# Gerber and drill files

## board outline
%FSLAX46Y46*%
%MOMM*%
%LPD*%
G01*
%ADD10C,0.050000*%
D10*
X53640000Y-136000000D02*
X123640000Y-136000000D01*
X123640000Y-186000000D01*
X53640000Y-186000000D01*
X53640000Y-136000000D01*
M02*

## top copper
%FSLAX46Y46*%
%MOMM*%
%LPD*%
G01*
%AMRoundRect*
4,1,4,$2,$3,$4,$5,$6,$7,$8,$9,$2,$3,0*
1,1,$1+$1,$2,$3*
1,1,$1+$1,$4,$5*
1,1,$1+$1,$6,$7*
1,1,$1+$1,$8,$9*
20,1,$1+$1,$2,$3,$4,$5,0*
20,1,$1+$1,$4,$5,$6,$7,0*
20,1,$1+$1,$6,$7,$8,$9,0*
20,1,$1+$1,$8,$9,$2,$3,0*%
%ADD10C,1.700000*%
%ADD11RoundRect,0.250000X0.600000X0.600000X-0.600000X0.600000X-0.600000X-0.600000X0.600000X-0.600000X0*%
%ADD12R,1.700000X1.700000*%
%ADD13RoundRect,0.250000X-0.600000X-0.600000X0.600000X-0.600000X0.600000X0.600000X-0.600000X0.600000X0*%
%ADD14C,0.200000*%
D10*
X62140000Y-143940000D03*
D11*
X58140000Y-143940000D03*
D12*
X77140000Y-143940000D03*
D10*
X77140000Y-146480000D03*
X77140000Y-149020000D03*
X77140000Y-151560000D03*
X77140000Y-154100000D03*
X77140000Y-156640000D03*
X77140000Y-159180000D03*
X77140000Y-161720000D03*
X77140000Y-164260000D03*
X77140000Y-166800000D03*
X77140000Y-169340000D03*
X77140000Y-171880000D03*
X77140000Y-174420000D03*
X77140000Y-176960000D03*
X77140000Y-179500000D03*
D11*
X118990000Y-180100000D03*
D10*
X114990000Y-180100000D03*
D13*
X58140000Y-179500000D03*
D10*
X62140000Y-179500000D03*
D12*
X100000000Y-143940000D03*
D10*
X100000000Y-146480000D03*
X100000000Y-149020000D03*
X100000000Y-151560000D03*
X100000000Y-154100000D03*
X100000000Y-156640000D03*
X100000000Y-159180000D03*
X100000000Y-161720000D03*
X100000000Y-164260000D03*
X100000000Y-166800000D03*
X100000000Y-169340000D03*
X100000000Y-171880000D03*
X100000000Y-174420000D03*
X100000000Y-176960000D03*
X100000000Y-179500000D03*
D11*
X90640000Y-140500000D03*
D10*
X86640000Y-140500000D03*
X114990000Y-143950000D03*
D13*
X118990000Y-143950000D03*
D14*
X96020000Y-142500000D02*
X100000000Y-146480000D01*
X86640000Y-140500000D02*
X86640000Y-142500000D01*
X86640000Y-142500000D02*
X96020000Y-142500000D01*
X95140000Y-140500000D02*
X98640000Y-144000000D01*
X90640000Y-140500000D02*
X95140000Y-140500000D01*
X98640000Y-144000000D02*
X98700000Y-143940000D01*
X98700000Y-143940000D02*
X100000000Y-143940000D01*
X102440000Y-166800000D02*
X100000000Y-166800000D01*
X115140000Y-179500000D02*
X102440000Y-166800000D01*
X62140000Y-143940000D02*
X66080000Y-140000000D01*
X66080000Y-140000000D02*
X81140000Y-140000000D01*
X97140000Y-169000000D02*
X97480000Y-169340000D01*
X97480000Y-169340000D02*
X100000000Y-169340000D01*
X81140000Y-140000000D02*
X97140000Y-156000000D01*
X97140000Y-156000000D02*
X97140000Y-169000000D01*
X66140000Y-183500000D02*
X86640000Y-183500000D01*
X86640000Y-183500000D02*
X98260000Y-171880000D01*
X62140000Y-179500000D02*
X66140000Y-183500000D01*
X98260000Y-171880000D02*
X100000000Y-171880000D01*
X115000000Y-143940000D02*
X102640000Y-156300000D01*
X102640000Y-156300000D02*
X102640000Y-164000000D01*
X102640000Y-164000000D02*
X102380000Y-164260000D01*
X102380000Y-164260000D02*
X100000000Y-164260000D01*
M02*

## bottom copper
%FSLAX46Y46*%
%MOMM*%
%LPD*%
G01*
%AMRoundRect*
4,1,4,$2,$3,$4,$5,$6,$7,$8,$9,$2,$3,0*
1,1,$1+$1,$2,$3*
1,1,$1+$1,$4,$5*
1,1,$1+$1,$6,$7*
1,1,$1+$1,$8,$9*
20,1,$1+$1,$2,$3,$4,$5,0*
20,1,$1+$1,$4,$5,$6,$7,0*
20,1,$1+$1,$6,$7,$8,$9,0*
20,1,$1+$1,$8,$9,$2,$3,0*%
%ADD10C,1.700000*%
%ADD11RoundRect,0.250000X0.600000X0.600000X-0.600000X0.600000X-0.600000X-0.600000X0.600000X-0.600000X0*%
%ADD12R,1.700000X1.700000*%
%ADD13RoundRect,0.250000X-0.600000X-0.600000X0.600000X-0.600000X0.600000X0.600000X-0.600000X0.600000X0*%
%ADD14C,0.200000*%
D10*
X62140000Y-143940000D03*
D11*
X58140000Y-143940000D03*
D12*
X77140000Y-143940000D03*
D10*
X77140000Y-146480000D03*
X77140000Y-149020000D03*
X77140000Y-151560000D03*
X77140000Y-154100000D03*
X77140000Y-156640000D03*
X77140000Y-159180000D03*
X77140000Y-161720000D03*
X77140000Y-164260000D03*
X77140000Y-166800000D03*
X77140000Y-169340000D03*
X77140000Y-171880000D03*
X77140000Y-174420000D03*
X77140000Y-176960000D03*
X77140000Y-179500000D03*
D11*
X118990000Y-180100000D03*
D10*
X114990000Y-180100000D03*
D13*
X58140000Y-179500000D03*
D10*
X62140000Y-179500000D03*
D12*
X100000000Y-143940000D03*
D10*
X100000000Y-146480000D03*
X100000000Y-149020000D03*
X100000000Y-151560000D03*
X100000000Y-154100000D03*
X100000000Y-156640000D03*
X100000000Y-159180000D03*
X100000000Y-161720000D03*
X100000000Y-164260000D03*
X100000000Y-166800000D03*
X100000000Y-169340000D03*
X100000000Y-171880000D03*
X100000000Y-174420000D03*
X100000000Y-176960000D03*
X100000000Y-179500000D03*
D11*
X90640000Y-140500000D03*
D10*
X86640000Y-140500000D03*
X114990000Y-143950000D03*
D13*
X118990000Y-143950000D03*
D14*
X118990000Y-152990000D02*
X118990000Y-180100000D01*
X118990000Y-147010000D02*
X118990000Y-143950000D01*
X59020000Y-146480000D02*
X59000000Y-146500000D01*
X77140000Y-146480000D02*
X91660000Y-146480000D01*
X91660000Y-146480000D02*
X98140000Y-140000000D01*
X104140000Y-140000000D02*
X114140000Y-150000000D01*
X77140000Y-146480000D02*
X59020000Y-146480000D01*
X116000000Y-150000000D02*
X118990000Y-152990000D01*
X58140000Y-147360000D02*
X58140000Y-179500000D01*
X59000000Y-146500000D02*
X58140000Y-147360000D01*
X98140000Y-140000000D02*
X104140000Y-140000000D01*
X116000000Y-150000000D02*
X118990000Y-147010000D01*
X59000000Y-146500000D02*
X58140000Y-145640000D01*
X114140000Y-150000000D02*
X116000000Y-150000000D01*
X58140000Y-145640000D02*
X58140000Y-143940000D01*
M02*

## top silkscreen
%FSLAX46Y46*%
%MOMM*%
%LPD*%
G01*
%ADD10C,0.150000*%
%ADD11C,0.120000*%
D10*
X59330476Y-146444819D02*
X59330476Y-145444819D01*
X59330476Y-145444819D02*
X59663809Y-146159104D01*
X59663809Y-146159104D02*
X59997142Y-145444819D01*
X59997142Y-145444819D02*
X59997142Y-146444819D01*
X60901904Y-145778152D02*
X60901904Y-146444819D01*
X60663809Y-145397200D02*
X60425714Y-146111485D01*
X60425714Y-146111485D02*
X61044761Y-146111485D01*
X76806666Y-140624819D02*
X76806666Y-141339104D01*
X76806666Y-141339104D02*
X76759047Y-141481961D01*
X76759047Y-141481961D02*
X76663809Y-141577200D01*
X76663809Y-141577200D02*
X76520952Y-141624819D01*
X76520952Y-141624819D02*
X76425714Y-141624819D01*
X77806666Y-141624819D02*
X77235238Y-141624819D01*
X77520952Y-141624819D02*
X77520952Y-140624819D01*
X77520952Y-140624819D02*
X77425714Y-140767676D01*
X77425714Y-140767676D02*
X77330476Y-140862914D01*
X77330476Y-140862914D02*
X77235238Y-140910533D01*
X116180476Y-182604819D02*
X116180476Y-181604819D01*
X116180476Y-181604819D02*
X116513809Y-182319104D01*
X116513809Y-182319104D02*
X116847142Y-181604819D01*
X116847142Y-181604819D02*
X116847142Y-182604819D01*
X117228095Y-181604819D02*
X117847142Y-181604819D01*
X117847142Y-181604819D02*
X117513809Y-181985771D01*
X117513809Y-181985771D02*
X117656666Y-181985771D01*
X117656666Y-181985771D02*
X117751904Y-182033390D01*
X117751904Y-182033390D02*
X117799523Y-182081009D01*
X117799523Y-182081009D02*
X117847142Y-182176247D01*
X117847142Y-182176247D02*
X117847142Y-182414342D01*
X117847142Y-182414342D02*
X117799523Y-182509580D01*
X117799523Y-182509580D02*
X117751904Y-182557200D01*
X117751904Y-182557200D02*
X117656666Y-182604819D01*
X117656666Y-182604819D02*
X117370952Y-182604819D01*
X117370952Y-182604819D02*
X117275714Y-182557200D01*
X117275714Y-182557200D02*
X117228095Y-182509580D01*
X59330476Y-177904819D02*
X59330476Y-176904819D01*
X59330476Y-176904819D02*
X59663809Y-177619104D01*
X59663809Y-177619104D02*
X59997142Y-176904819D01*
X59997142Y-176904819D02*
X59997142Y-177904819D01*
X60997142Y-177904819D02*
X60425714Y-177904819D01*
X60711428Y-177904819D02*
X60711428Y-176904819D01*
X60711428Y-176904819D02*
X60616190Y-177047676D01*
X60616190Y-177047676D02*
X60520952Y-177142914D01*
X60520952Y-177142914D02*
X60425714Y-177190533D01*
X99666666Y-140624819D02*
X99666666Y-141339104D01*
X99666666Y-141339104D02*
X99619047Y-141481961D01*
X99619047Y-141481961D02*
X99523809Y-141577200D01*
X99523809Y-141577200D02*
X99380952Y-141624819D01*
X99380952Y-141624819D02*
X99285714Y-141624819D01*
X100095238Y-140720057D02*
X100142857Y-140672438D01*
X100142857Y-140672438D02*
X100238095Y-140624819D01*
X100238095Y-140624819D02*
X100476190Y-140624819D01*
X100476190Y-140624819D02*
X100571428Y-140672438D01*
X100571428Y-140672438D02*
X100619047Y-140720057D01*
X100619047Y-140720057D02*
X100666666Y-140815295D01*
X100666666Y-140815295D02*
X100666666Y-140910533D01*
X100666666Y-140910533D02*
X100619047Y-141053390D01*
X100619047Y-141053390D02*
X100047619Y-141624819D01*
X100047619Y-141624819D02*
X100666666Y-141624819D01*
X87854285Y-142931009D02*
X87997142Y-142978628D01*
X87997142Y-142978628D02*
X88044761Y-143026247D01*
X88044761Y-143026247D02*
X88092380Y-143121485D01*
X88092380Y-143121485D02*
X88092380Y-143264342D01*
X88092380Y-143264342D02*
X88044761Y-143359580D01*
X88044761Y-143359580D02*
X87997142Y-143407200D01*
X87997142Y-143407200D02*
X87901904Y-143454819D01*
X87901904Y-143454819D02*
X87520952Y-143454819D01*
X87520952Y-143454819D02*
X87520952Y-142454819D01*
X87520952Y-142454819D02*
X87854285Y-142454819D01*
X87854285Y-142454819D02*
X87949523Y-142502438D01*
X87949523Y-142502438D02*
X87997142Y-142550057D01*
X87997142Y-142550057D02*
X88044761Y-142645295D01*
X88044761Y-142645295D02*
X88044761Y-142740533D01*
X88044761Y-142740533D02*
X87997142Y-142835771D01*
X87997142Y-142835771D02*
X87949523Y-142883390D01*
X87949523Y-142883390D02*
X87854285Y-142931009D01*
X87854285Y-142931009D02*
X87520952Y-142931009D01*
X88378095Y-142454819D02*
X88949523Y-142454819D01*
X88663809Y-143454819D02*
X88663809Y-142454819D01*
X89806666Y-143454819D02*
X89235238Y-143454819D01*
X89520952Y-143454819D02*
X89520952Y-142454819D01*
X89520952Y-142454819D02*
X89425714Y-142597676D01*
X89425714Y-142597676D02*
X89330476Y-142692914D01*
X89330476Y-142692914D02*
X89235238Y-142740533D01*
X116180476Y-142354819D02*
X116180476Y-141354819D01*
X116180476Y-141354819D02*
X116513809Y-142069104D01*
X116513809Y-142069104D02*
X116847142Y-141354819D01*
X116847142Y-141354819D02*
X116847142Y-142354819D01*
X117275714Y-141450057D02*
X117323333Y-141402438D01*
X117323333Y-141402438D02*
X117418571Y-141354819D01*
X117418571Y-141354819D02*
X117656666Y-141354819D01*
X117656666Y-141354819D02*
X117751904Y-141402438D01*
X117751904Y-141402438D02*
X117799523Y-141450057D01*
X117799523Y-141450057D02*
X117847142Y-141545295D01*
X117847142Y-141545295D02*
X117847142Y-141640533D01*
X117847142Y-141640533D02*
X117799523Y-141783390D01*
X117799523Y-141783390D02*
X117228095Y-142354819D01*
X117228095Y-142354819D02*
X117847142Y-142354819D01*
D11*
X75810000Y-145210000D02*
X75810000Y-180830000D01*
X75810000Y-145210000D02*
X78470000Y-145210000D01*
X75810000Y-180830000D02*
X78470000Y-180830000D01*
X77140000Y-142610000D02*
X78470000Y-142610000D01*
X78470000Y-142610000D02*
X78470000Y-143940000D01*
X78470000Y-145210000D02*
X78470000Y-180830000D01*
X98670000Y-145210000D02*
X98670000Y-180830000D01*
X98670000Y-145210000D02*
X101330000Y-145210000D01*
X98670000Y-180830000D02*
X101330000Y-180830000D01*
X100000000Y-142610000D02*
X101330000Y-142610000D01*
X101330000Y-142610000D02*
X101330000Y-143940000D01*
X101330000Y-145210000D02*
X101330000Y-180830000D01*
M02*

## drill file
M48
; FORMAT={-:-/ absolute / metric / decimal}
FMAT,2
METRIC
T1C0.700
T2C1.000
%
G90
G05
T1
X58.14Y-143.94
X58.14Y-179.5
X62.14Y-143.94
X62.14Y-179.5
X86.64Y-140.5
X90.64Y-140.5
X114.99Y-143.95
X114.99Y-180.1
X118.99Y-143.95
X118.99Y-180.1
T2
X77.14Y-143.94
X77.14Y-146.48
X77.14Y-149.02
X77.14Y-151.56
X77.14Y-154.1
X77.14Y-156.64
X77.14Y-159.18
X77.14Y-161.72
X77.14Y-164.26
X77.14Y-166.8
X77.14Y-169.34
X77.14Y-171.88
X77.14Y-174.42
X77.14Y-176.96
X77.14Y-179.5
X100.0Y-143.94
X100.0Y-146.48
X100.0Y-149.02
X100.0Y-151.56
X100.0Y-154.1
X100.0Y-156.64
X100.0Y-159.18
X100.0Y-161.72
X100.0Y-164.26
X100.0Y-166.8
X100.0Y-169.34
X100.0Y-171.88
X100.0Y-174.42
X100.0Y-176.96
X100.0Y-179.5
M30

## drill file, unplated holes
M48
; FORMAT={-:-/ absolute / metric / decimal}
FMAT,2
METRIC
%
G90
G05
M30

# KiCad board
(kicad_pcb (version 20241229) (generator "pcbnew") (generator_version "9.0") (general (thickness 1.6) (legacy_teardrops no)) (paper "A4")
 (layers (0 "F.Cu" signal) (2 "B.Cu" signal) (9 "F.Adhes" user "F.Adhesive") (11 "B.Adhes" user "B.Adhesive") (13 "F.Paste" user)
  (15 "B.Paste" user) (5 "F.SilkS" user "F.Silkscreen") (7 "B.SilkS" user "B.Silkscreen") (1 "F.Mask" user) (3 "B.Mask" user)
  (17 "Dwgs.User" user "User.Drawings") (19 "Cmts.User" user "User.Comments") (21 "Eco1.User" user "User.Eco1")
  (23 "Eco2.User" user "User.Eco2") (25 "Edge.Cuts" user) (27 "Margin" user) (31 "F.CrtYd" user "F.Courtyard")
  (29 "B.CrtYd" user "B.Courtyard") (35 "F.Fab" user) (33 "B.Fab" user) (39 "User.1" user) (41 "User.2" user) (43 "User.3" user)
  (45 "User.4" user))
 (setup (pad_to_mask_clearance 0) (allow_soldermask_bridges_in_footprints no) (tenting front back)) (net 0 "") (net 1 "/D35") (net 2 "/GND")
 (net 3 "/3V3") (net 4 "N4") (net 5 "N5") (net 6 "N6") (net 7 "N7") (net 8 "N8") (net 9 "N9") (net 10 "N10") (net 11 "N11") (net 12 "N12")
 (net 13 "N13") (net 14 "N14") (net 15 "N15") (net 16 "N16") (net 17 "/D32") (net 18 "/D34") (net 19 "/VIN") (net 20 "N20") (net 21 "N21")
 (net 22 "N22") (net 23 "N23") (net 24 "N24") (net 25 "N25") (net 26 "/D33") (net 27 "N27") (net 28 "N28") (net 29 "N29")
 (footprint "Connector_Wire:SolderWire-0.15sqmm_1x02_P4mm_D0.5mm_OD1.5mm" (layer "F.Cu") (at 62.14 143.94 180)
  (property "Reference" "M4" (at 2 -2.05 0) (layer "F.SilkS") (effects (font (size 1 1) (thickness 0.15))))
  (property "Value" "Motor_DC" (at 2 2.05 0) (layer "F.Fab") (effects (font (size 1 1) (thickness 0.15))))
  (pad "1" thru_hole circle (at 0 0 180) (size 1.7 1.7) (drill 0.7) (layers "*.Cu" "*.Mask") (remove_unused_layers no) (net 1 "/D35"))
  (pad "2" thru_hole roundrect (at 4 0 180) (size 1.7 1.7) (drill 0.7) (layers "*.Cu" "*.Mask") (remove_unused_layers no)
   (roundrect_rratio 0.1470588235) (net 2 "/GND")))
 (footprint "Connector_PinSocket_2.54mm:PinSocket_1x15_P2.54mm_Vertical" (layer "F.Cu") (at 77.14 143.94)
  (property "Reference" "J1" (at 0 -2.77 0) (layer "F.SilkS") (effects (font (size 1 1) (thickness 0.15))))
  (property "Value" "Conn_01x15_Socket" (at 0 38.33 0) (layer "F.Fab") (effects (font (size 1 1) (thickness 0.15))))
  (fp_line (start -1.33 1.27) (end -1.33 36.89) (stroke (width 0.12) (type solid)) (layer "F.SilkS"))
  (fp_line (start -1.33 1.27) (end 1.33 1.27) (stroke (width 0.12) (type solid)) (layer "F.SilkS"))
  (fp_line (start -1.33 36.89) (end 1.33 36.89) (stroke (width 0.12) (type solid)) (layer "F.SilkS"))
  (fp_line (start 0 -1.33) (end 1.33 -1.33) (stroke (width 0.12) (type solid)) (layer "F.SilkS"))
  (fp_line (start 1.33 -1.33) (end 1.33 0) (stroke (width 0.12) (type solid)) (layer "F.SilkS"))
  (fp_line (start 1.33 1.27) (end 1.33 36.89) (stroke (width 0.12) (type solid)) (layer "F.SilkS"))
  (pad "1" thru_hole rect (at 0 0) (size 1.7 1.7) (drill 1) (layers "*.Cu" "*.Mask") (remove_unused_layers no) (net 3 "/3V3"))
  (pad "2" thru_hole circle (at 0 2.54) (size 1.7 1.7) (drill 1) (layers "*.Cu" "*.Mask") (remove_unused_layers no) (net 2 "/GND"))
  (pad "3" thru_hole circle (at 0 5.08) (size 1.7 1.7) (drill 1) (layers "*.Cu" "*.Mask") (remove_unused_layers no) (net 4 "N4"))
  (pad "4" thru_hole circle (at 0 7.62) (size 1.7 1.7) (drill 1) (layers "*.Cu" "*.Mask") (remove_unused_layers no) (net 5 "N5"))
  (pad "5" thru_hole circle (at 0 10.16) (size 1.7 1.7) (drill 1) (layers "*.Cu" "*.Mask") (remove_unused_layers no) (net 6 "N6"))
  (pad "6" thru_hole circle (at 0 12.7) (size 1.7 1.7) (drill 1) (layers "*.Cu" "*.Mask") (remove_unused_layers no) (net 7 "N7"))
  (pad "7" thru_hole circle (at 0 15.24) (size 1.7 1.7) (drill 1) (layers "*.Cu" "*.Mask") (remove_unused_layers no) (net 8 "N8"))
  (pad "8" thru_hole circle (at 0 17.78) (size 1.7 1.7) (drill 1) (layers "*.Cu" "*.Mask") (remove_unused_layers no) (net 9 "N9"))
  (pad "9" thru_hole circle (at 0 20.32) (size 1.7 1.7) (drill 1) (layers "*.Cu" "*.Mask") (remove_unused_layers no) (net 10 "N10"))
  (pad "10" thru_hole circle (at 0 22.86) (size 1.7 1.7) (drill 1) (layers "*.Cu" "*.Mask") (remove_unused_layers no) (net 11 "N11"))
  (pad "11" thru_hole circle (at 0 25.4) (size 1.7 1.7) (drill 1) (layers "*.Cu" "*.Mask") (remove_unused_layers no) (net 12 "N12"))
  (pad "12" thru_hole circle (at 0 27.94) (size 1.7 1.7) (drill 1) (layers "*.Cu" "*.Mask") (remove_unused_layers no) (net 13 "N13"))
  (pad "13" thru_hole circle (at 0 30.48) (size 1.7 1.7) (drill 1) (layers "*.Cu" "*.Mask") (remove_unused_layers no) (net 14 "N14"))
  (pad "14" thru_hole circle (at 0 33.02) (size 1.7 1.7) (drill 1) (layers "*.Cu" "*.Mask") (remove_unused_layers no) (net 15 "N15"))
  (pad "15" thru_hole circle (at 0 35.56) (size 1.7 1.7) (drill 1) (layers "*.Cu" "*.Mask") (remove_unused_layers no) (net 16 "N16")))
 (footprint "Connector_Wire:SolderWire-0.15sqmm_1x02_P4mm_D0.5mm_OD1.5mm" (layer "F.Cu") (at 118.99 180.1 180)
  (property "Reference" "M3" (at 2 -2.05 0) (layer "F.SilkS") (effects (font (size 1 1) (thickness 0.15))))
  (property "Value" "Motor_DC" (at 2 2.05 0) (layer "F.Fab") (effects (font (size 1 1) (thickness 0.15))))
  (pad "1" thru_hole roundrect (at 0 0 180) (size 1.7 1.7) (drill 0.7) (layers "*.Cu" "*.Mask") (remove_unused_layers no)
   (roundrect_rratio 0.147059) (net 2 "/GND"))
  (pad "2" thru_hole circle (at 4 0 180) (size 1.7 1.7) (drill 0.7) (layers "*.Cu" "*.Mask") (remove_unused_layers no) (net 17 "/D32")))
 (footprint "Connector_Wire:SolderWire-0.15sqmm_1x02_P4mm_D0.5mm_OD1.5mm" (layer "F.Cu") (at 58.14 179.5)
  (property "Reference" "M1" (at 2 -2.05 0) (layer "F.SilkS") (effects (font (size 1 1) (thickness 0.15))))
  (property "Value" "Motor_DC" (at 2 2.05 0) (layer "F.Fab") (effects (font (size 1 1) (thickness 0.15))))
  (pad "1" thru_hole roundrect (at 0 0) (size 1.7 1.7) (drill 0.7) (layers "*.Cu" "*.Mask") (remove_unused_layers no)
   (roundrect_rratio 0.147059) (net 2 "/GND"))
  (pad "2" thru_hole circle (at 4 0) (size 1.7 1.7) (drill 0.7) (layers "*.Cu" "*.Mask") (remove_unused_layers no) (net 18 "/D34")))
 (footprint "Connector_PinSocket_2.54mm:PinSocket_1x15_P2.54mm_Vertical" (layer "F.Cu") (at 100 143.94)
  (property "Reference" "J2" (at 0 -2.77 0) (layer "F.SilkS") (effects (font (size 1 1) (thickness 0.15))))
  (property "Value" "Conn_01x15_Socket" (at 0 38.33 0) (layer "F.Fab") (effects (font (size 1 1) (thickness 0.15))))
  (fp_line (start -1.33 1.27) (end -1.33 36.89) (stroke (width 0.12) (type solid)) (layer "F.SilkS"))
  (fp_line (start -1.33 1.27) (end 1.33 1.27) (stroke (width 0.12) (type solid)) (layer "F.SilkS"))
  (fp_line (start -1.33 36.89) (end 1.33 36.89) (stroke (width 0.12) (type solid)) (layer "F.SilkS"))
  (fp_line (start 0 -1.33) (end 1.33 -1.33) (stroke (width 0.12) (type solid)) (layer "F.SilkS"))
  (fp_line (start 1.33 -1.33) (end 1.33 0) (stroke (width 0.12) (type solid)) (layer "F.SilkS"))
  (fp_line (start 1.33 1.27) (end 1.33 36.89) (stroke (width 0.12) (type solid)) (layer "F.SilkS"))
  (pad "1" thru_hole rect (at 0 0) (size 1.7 1.7) (drill 1) (layers "*.Cu" "*.Mask") (remove_unused_layers no) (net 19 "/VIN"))
  (pad "2" thru_hole circle (at 0 2.54) (size 1.7 1.7) (drill 1) (layers "*.Cu" "*.Mask") (remove_unused_layers no) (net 2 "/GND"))
  (pad "3" thru_hole circle (at 0 5.08) (size 1.7 1.7) (drill 1) (layers "*.Cu" "*.Mask") (remove_unused_layers no) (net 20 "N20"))
  (pad "4" thru_hole circle (at 0 7.62) (size 1.7 1.7) (drill 1) (layers "*.Cu" "*.Mask") (remove_unused_layers no) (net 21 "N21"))
  (pad "5" thru_hole circle (at 0 10.16) (size 1.7 1.7) (drill 1) (layers "*.Cu" "*.Mask") (remove_unused_layers no) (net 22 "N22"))
  (pad "6" thru_hole circle (at 0 12.7) (size 1.7 1.7) (drill 1) (layers "*.Cu" "*.Mask") (remove_unused_layers no) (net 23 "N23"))
  (pad "7" thru_hole circle (at 0 15.24) (size 1.7 1.7) (drill 1) (layers "*.Cu" "*.Mask") (remove_unused_layers no) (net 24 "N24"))
  (pad "8" thru_hole circle (at 0 17.78) (size 1.7 1.7) (drill 1) (layers "*.Cu" "*.Mask") (remove_unused_layers no) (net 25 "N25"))
  (pad "9" thru_hole circle (at 0 20.32) (size 1.7 1.7) (drill 1) (layers "*.Cu" "*.Mask") (remove_unused_layers no) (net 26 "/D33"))
  (pad "10" thru_hole circle (at 0 22.86) (size 1.7 1.7) (drill 1) (layers "*.Cu" "*.Mask") (remove_unused_layers no) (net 17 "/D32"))
  (pad "11" thru_hole circle (at 0 25.4) (size 1.7 1.7) (drill 1) (layers "*.Cu" "*.Mask") (remove_unused_layers no) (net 1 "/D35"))
  (pad "12" thru_hole circle (at 0 27.94) (size 1.7 1.7) (drill 1) (layers "*.Cu" "*.Mask") (remove_unused_layers no) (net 18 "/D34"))
  (pad "13" thru_hole circle (at 0 30.48) (size 1.7 1.7) (drill 1) (layers "*.Cu" "*.Mask") (remove_unused_layers no) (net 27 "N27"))
  (pad "14" thru_hole circle (at 0 33.02) (size 1.7 1.7) (drill 1) (layers "*.Cu" "*.Mask") (remove_unused_layers no) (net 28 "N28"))
  (pad "15" thru_hole circle (at 0 35.56) (size 1.7 1.7) (drill 1) (layers "*.Cu" "*.Mask") (remove_unused_layers no) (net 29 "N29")))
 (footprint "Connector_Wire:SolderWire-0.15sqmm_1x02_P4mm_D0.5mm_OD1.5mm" (layer "F.Cu") (at 90.64 140.5 180)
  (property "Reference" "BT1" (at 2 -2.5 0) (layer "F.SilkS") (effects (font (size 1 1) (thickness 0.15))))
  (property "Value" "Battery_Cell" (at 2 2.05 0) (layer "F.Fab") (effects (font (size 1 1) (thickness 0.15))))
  (pad "1" thru_hole roundrect (at 0 0 180) (size 1.7 1.7) (drill 0.7) (layers "*.Cu" "*.Mask") (remove_unused_layers no)
   (roundrect_rratio 0.147059) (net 19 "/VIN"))
  (pad "2" thru_hole circle (at 4 0 180) (size 1.7 1.7) (drill 0.7) (layers "*.Cu" "*.Mask") (remove_unused_layers no) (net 2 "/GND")))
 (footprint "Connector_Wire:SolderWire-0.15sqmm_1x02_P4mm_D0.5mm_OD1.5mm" (layer "F.Cu") (at 114.99 143.95)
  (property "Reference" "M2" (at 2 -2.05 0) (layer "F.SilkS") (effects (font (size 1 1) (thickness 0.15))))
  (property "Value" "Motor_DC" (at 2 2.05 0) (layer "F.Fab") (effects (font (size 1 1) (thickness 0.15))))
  (pad "1" thru_hole circle (at 0 0) (size 1.7 1.7) (drill 0.7) (layers "*.Cu" "*.Mask") (remove_unused_layers no) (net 26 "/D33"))
  (pad "2" thru_hole roundrect (at 4 0) (size 1.7 1.7) (drill 0.7) (layers "*.Cu" "*.Mask") (remove_unused_layers no)
   (roundrect_rratio 0.1470588235) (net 2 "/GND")))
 (gr_rect (start 53.64 136) (end 123.64 186) (stroke (width 0.05) (type default)) (fill no) (layer "Edge.Cuts"))
 (segment (start 96.02 142.5) (end 100 146.48) (width 0.2) (layer "F.Cu") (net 2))
 (segment (start 86.64 140.5) (end 86.64 142.5) (width 0.2) (layer "F.Cu") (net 2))
 (segment (start 86.64 142.5) (end 96.02 142.5) (width 0.2) (layer "F.Cu") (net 2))
 (segment (start 118.99 152.99) (end 118.99 180.1) (width 0.2) (layer "B.Cu") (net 2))
 (segment (start 118.99 147.01) (end 118.99 143.95) (width 0.2) (layer "B.Cu") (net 2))
 (segment (start 59.02 146.48) (end 59 146.5) (width 0.2) (layer "B.Cu") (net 2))
 (segment (start 77.14 146.48) (end 91.66 146.48) (width 0.2) (layer "B.Cu") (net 2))
 (segment (start 91.66 146.48) (end 98.14 140) (width 0.2) (layer "B.Cu") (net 2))
 (segment (start 104.14 140) (end 114.14 150) (width 0.2) (layer "B.Cu") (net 2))
 (segment (start 77.14 146.48) (end 59.02 146.48) (width 0.2) (layer "B.Cu") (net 2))
 (segment (start 116 150) (end 118.99 152.99) (width 0.2) (layer "B.Cu") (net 2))
 (segment (start 58.14 147.36) (end 58.14 179.5) (width 0.2) (layer "B.Cu") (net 2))
 (segment (start 59 146.5) (end 58.14 147.36) (width 0.2) (layer "B.Cu") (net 2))
 (segment (start 98.14 140) (end 104.14 140) (width 0.2) (layer "B.Cu") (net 2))
 (segment (start 116 150) (end 118.99 147.01) (width 0.2) (layer "B.Cu") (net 2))
 (segment (start 59 146.5) (end 58.14 145.64) (width 0.2) (layer "B.Cu") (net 2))
 (segment (start 114.14 150) (end 116 150) (width 0.2) (layer "B.Cu") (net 2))
 (segment (start 58.14 145.64) (end 58.14 143.94) (width 0.2) (layer "B.Cu") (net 2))
 (segment (start 95.14 140.5) (end 98.64 144) (width 0.2) (layer "F.Cu") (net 19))
 (segment (start 90.64 140.5) (end 95.14 140.5) (width 0.2) (layer "F.Cu") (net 19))
 (segment (start 98.64 144) (end 98.7 143.94) (width 0.2) (layer "F.Cu") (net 19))
 (segment (start 98.7 143.94) (end 100 143.94) (width 0.2) (layer "F.Cu") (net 19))
 (segment (start 102.44 166.8) (end 100 166.8) (width 0.2) (layer "F.Cu") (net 17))
 (segment (start 115.14 179.5) (end 102.44 166.8) (width 0.2) (layer "F.Cu") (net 17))
 (segment (start 62.14 143.94) (end 66.08 140) (width 0.2) (layer "F.Cu") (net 1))
 (segment (start 66.08 140) (end 81.14 140) (width 0.2) (layer "F.Cu") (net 1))
 (segment (start 97.14 169) (end 97.48 169.34) (width 0.2) (layer "F.Cu") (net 1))
 (segment (start 97.48 169.34) (end 100 169.34) (width 0.2) (layer "F.Cu") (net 1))
 (segment (start 81.14 140) (end 97.14 156) (width 0.2) (layer "F.Cu") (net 1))
 (segment (start 97.14 156) (end 97.14 169) (width 0.2) (layer "F.Cu") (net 1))
 (segment (start 66.14 183.5) (end 86.64 183.5) (width 0.2) (layer "F.Cu") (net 18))
 (segment (start 86.64 183.5) (end 98.26 171.88) (width 0.2) (layer "F.Cu") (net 18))
 (segment (start 62.14 179.5) (end 66.14 183.5) (width 0.2) (layer "F.Cu") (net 18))
 (segment (start 98.26 171.88) (end 100 171.88) (width 0.2) (layer "F.Cu") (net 18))
 (segment (start 115 143.94) (end 102.64 156.3) (width 0.2) (layer "F.Cu") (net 26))
 (segment (start 102.64 156.3) (end 102.64 164) (width 0.2) (layer "F.Cu") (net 26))
 (segment (start 102.64 164) (end 102.38 164.26) (width 0.2) (layer "F.Cu") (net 26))
 (segment (start 102.38 164.26) (end 100 164.26) (width 0.2) (layer "F.Cu") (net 26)))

